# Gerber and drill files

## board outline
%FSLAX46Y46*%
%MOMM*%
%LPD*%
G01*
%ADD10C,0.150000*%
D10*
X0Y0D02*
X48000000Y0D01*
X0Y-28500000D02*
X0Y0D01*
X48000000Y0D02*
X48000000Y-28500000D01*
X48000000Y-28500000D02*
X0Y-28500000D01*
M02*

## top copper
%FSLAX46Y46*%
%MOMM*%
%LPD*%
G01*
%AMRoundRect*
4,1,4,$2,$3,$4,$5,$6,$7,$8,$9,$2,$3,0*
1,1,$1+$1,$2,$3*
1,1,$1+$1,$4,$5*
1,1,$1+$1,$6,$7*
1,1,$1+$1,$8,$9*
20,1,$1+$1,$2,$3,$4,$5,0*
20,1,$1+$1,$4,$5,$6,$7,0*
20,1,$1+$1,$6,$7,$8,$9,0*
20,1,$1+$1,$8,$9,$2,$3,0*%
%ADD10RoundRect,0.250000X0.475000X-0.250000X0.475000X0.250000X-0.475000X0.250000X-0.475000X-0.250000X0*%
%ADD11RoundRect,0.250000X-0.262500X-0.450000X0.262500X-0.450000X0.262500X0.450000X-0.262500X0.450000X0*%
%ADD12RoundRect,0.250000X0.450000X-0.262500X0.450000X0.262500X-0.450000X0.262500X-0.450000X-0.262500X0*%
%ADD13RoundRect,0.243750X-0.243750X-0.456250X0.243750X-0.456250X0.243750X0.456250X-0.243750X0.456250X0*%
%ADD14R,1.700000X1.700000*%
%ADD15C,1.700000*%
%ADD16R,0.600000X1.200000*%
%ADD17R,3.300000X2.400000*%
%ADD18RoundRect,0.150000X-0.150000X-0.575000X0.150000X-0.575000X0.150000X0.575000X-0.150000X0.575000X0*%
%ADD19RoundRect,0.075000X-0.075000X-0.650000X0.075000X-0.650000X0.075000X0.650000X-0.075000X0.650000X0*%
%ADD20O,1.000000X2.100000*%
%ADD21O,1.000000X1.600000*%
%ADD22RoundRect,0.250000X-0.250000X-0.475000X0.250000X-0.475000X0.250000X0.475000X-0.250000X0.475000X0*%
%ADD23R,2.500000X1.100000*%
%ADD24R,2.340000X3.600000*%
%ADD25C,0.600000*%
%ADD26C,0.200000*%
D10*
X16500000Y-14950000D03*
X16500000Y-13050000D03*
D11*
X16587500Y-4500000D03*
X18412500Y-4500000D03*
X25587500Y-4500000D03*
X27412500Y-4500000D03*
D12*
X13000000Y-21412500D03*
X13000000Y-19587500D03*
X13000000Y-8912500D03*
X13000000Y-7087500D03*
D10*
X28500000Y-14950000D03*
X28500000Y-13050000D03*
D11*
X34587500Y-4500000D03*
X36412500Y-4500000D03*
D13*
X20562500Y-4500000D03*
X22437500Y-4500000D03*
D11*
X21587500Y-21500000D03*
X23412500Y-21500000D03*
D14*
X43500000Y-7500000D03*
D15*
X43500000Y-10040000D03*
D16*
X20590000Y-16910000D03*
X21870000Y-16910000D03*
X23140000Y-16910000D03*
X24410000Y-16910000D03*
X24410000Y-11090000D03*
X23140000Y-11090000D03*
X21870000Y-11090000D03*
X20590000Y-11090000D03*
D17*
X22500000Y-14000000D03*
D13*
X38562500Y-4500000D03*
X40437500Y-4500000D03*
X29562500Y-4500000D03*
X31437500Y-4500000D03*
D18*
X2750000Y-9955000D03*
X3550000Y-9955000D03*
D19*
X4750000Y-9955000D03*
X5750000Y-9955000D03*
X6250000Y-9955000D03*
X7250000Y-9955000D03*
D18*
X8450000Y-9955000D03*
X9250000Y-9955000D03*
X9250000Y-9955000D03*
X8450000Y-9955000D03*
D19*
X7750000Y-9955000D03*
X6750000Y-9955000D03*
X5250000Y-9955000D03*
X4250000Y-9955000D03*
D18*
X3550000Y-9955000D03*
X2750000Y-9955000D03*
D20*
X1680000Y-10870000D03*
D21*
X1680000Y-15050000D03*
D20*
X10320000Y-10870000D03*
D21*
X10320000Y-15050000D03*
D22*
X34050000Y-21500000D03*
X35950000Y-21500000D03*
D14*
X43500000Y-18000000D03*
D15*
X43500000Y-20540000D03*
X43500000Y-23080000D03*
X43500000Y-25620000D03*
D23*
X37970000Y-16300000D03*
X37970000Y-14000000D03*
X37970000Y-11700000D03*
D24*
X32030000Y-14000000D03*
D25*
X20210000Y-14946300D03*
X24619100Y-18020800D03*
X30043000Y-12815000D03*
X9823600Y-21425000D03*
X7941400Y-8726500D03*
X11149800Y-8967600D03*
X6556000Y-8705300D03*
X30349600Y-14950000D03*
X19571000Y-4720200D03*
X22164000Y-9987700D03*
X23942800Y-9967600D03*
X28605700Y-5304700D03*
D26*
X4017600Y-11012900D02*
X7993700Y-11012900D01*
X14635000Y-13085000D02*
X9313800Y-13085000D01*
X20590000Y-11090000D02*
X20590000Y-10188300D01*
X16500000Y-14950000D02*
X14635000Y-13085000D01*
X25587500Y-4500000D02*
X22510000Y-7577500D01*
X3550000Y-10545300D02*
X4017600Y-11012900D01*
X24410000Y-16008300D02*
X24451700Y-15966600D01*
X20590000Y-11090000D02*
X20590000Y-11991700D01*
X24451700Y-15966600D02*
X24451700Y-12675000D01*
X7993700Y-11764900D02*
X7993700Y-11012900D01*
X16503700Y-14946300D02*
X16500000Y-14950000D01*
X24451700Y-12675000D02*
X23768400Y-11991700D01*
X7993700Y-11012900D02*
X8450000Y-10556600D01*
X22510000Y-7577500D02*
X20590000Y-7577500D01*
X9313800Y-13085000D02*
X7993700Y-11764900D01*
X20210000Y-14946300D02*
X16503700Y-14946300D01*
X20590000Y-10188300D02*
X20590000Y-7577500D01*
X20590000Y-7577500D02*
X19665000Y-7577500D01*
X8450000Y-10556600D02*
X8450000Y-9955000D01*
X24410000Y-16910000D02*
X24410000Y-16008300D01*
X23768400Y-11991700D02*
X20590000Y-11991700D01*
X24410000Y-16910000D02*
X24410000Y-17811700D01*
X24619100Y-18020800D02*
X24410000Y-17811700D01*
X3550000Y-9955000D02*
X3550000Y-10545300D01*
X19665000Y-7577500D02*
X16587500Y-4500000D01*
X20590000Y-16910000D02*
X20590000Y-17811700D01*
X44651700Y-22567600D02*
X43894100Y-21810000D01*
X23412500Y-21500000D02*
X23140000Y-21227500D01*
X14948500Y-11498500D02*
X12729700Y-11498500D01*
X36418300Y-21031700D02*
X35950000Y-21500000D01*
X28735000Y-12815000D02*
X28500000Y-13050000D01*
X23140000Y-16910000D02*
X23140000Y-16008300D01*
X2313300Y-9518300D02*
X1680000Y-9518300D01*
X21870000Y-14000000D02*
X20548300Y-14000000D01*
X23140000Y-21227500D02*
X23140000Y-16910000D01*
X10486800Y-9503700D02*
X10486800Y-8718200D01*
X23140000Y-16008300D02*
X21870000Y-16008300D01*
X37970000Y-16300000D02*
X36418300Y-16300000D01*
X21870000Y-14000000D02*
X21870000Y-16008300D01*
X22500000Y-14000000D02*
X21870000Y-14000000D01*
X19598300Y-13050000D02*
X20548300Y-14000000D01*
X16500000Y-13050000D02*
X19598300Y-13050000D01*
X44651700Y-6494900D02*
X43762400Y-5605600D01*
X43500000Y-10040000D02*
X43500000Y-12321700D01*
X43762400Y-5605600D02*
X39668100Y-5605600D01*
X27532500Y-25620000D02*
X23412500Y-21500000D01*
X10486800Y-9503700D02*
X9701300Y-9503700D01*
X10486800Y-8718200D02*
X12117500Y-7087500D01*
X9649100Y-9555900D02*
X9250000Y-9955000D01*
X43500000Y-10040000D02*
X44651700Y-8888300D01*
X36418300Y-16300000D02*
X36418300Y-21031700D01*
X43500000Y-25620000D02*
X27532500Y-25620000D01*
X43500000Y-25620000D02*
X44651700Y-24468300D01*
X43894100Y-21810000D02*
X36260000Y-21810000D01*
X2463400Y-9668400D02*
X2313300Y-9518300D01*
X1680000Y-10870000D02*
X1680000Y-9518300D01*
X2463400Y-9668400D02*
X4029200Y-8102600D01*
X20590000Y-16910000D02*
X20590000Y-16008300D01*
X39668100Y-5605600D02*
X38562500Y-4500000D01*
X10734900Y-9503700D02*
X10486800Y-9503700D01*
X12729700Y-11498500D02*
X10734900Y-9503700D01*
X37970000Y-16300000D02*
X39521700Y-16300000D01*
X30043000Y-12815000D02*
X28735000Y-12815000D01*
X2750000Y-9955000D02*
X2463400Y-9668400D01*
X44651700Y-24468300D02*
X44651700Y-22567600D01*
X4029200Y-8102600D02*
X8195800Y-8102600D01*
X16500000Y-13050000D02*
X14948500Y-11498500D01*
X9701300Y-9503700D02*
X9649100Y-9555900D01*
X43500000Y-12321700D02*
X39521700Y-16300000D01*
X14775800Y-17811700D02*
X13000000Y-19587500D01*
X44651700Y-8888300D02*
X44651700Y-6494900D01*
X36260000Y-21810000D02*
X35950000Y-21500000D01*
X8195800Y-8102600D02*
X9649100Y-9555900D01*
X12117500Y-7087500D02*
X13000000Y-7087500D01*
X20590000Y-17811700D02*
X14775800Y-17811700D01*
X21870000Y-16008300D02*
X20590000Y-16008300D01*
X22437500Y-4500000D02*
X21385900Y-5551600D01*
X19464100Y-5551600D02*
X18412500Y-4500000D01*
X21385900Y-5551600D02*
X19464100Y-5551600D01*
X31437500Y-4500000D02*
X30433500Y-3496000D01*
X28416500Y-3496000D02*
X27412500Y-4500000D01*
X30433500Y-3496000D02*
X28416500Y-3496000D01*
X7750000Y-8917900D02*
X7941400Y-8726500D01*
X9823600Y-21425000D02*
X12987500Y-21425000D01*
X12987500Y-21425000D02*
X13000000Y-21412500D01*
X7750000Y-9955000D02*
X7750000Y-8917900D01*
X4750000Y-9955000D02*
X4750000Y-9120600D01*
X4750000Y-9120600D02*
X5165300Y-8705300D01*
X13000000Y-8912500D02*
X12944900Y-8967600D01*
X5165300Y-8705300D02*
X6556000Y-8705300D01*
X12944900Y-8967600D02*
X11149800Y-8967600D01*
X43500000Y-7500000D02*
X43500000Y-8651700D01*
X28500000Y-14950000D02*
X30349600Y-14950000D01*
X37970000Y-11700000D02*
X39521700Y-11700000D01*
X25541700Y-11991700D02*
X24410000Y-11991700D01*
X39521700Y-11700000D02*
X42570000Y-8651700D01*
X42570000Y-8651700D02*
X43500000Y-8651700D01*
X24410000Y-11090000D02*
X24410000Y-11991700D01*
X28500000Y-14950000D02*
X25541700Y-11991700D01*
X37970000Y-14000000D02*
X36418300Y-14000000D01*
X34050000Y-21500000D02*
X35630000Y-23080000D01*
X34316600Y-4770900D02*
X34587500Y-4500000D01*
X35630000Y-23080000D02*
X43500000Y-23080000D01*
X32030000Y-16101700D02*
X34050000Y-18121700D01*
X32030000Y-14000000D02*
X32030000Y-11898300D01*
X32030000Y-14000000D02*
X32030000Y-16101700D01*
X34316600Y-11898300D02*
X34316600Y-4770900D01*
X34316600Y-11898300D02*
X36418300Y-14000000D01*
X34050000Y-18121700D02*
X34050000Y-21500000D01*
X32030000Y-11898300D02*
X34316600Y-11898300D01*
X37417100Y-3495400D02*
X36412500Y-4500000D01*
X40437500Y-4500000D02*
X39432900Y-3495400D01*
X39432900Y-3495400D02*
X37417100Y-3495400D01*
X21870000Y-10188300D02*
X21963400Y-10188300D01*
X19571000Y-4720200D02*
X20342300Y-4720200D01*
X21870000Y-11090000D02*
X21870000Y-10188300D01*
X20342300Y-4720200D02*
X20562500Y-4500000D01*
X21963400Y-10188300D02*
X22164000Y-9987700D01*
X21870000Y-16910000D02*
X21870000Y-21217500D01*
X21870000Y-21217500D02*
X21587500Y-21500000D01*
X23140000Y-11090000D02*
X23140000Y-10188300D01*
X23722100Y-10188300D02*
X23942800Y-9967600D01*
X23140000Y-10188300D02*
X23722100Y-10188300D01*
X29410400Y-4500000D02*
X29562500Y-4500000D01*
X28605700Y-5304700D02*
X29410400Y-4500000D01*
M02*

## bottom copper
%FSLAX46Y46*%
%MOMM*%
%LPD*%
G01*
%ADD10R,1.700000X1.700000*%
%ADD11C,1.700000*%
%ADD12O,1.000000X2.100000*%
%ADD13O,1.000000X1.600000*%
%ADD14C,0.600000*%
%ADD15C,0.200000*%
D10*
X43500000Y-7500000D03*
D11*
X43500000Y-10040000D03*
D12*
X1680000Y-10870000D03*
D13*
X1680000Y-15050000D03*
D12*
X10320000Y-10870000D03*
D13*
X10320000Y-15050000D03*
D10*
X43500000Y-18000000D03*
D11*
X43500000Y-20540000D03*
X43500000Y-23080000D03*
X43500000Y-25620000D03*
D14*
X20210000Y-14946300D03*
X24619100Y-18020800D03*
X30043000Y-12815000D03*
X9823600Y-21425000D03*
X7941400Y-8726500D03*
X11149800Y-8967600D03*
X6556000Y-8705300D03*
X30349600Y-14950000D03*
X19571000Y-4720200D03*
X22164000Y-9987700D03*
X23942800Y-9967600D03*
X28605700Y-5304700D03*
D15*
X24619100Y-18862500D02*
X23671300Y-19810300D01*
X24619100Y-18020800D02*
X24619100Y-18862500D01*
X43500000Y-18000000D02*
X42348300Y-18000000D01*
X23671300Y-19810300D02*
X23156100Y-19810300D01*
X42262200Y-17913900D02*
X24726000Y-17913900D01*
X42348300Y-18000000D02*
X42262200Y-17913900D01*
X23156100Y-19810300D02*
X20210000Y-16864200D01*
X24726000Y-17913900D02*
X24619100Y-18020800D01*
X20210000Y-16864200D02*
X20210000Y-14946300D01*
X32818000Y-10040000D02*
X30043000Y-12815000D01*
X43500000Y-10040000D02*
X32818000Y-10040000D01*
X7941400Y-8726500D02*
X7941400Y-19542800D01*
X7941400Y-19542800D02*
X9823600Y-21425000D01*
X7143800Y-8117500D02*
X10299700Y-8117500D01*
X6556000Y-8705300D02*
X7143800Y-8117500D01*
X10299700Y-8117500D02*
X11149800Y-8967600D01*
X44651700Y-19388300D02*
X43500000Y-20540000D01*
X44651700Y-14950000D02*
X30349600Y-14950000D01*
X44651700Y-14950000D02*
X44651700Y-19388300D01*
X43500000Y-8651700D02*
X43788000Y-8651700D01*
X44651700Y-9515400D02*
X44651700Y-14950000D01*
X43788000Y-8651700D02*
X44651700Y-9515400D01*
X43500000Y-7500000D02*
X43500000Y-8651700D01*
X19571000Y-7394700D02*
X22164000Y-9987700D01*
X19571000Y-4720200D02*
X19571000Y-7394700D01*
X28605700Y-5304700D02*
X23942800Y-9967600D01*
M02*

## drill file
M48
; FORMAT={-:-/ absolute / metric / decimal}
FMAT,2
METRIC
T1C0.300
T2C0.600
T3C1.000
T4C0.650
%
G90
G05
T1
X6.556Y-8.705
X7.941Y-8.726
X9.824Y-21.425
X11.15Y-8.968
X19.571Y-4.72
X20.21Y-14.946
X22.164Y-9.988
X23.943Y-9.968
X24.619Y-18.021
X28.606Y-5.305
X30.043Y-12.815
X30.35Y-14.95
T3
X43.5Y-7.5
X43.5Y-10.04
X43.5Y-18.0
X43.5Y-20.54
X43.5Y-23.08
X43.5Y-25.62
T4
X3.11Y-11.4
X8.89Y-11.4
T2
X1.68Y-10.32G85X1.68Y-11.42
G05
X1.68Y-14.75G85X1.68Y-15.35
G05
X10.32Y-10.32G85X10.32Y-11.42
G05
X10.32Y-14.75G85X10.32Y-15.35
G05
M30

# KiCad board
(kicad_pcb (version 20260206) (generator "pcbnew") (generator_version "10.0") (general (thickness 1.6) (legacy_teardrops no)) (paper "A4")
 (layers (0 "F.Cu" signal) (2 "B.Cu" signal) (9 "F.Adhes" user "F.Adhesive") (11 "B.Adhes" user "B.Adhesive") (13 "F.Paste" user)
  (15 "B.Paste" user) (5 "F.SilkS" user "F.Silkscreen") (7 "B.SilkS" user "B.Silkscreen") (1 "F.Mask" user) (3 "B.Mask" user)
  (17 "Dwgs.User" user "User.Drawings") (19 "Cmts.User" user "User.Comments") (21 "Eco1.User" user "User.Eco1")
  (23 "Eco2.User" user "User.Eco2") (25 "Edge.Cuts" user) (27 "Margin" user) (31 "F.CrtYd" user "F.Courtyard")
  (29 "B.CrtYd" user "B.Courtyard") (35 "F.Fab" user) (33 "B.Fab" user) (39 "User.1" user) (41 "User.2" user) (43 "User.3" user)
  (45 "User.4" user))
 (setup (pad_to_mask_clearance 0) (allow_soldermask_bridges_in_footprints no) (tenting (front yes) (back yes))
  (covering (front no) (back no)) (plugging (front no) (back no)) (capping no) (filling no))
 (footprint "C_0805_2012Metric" (layer "F.Cu") (at 16.5 14 90)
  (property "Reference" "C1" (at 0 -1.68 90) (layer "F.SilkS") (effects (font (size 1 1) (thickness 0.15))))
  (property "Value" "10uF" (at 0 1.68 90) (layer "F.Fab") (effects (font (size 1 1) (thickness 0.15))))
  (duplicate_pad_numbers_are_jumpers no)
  (pad "1" smd roundrect (at -0.95 0 90) (size 1 1.45) (layers "F.Cu" "F.Mask" "F.Paste") (roundrect_rratio 0.25) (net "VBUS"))
  (pad "2" smd roundrect (at 0.95 0 90) (size 1 1.45) (layers "F.Cu" "F.Mask" "F.Paste") (roundrect_rratio 0.25) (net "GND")))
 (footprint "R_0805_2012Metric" (layer "F.Cu") (at 17.5 4.5)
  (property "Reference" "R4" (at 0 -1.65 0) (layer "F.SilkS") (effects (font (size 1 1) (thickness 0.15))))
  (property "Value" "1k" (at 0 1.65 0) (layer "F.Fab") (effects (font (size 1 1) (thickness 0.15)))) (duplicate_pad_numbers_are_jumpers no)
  (pad "1" smd roundrect (at -0.9125 0) (size 1.025 1.4) (layers "F.Cu" "F.Mask" "F.Paste") (roundrect_rratio 0.243902) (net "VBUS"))
  (pad "2" smd roundrect (at 0.9125 0) (size 1.025 1.4) (layers "F.Cu" "F.Mask" "F.Paste") (roundrect_rratio 0.243902) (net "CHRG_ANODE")))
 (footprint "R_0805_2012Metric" (layer "F.Cu") (at 26.5 4.5)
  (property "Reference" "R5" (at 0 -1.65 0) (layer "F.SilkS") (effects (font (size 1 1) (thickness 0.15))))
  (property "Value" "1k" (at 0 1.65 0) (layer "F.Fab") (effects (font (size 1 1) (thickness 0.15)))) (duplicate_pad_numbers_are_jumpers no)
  (pad "1" smd roundrect (at -0.9125 0) (size 1.025 1.4) (layers "F.Cu" "F.Mask" "F.Paste") (roundrect_rratio 0.243902) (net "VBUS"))
  (pad "2" smd roundrect (at 0.9125 0) (size 1.025 1.4) (layers "F.Cu" "F.Mask" "F.Paste") (roundrect_rratio 0.243902) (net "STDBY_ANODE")))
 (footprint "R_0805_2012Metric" (layer "F.Cu") (at 13 20.5 90)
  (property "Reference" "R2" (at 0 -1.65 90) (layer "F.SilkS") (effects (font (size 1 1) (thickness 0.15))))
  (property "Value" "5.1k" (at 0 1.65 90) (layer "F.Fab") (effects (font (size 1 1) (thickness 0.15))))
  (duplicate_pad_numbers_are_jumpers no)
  (pad "1" smd roundrect (at -0.9125 0 90) (size 1.025 1.4) (layers "F.Cu" "F.Mask" "F.Paste") (roundrect_rratio 0.243902) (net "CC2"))
  (pad "2" smd roundrect (at 0.9125 0 90) (size 1.025 1.4) (layers "F.Cu" "F.Mask" "F.Paste") (roundrect_rratio 0.243902) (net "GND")))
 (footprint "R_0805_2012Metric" (layer "F.Cu") (at 13 8 90)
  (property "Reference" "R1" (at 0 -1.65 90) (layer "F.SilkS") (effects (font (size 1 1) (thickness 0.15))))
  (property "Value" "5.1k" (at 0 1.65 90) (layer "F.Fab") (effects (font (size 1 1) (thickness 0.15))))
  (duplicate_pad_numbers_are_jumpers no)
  (pad "1" smd roundrect (at -0.9125 0 90) (size 1.025 1.4) (layers "F.Cu" "F.Mask" "F.Paste") (roundrect_rratio 0.243902) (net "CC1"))
  (pad "2" smd roundrect (at 0.9125 0 90) (size 1.025 1.4) (layers "F.Cu" "F.Mask" "F.Paste") (roundrect_rratio 0.243902) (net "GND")))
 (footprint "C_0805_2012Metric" (layer "F.Cu") (at 28.5 14 90)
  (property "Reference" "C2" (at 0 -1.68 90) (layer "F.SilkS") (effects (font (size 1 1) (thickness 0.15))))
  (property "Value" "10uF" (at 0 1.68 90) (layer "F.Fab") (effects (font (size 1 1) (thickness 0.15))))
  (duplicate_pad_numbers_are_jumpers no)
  (pad "1" smd roundrect (at -0.95 0 90) (size 1 1.45) (layers "F.Cu" "F.Mask" "F.Paste") (roundrect_rratio 0.25) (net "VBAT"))
  (pad "2" smd roundrect (at 0.95 0 90) (size 1 1.45) (layers "F.Cu" "F.Mask" "F.Paste") (roundrect_rratio 0.25) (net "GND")))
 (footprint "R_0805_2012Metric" (layer "F.Cu") (at 35.5 4.5)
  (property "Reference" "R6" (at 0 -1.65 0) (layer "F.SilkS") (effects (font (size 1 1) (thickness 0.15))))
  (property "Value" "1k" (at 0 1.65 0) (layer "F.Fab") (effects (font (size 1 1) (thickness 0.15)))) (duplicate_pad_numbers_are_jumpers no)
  (pad "1" smd roundrect (at -0.9125 0) (size 1.025 1.4) (layers "F.Cu" "F.Mask" "F.Paste") (roundrect_rratio 0.243902) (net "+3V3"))
  (pad "2" smd roundrect (at 0.9125 0) (size 1.025 1.4) (layers "F.Cu" "F.Mask" "F.Paste") (roundrect_rratio 0.243902) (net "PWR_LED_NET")))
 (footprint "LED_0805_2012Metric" (layer "F.Cu") (at 21.5 4.5)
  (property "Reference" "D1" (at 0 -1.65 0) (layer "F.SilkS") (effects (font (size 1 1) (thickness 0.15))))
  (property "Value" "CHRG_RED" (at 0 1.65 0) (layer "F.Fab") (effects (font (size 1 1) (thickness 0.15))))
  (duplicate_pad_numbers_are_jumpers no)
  (pad "1" smd roundrect (at -0.9375 0) (size 0.975 1.4) (layers "F.Cu" "F.Mask" "F.Paste") (roundrect_rratio 0.25) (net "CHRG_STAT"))
  (pad "2" smd roundrect (at 0.9375 0) (size 0.975 1.4) (layers "F.Cu" "F.Mask" "F.Paste") (roundrect_rratio 0.25) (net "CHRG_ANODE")))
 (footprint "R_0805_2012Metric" (layer "F.Cu") (at 22.5 21.5)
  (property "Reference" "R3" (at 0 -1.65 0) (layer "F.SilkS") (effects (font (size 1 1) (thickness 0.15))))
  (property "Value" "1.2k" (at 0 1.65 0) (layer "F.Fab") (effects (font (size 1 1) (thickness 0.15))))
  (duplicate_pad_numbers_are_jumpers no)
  (pad "1" smd roundrect (at -0.9125 0) (size 1.025 1.4) (layers "F.Cu" "F.Mask" "F.Paste") (roundrect_rratio 0.243902) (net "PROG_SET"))
  (pad "2" smd roundrect (at 0.9125 0) (size 1.025 1.4) (layers "F.Cu" "F.Mask" "F.Paste") (roundrect_rratio 0.243902) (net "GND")))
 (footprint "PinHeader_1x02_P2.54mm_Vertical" (layer "F.Cu") (at 43.5 7.5)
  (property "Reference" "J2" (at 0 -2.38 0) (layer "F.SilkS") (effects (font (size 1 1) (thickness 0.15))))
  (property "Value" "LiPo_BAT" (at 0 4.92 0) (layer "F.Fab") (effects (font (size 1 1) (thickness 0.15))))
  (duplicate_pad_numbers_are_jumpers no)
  (pad "1" thru_hole rect (at 0 0) (size 1.7 1.7) (drill 1) (layers "*.Cu" "*.Mask") (remove_unused_layers no) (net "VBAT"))
  (pad "2" thru_hole circle (at 0 2.54) (size 1.7 1.7) (drill 1) (layers "*.Cu" "*.Mask") (remove_unused_layers no) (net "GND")))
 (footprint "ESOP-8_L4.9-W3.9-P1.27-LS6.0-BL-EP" (layer "F.Cu") (at 22.5 14)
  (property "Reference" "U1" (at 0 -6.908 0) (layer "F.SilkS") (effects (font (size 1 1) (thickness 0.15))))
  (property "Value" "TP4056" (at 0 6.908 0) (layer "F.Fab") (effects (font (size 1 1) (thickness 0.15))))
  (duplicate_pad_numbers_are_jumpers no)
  (pad "1" smd rect (at -1.91 2.91) (size 0.6 1.2) (layers "F.Cu" "F.Mask" "F.Paste") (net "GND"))
  (pad "2" smd rect (at -0.63 2.91) (size 0.6 1.2) (layers "F.Cu" "F.Mask" "F.Paste") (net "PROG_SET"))
  (pad "3" smd rect (at 0.64 2.91) (size 0.6 1.2) (layers "F.Cu" "F.Mask" "F.Paste") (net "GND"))
  (pad "4" smd rect (at 1.91 2.91) (size 0.6 1.2) (layers "F.Cu" "F.Mask" "F.Paste") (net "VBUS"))
  (pad "5" smd rect (at 1.91 -2.91) (size 0.6 1.2) (layers "F.Cu" "F.Mask" "F.Paste") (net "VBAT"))
  (pad "6" smd rect (at 0.64 -2.91) (size 0.6 1.2) (layers "F.Cu" "F.Mask" "F.Paste") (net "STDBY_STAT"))
  (pad "7" smd rect (at -0.63 -2.91) (size 0.6 1.2) (layers "F.Cu" "F.Mask" "F.Paste") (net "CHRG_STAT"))
  (pad "8" smd rect (at -1.91 -2.91) (size 0.6 1.2) (layers "F.Cu" "F.Mask" "F.Paste") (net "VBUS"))
  (pad "9" smd rect (at 0 0 180) (size 3.3 2.4) (layers "F.Cu" "F.Mask" "F.Paste") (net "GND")))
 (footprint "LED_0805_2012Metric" (layer "F.Cu") (at 39.5 4.5)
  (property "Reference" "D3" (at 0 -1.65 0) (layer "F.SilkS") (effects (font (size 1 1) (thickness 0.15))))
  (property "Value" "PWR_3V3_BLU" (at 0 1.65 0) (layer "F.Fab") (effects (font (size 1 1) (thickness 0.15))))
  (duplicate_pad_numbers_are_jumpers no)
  (pad "1" smd roundrect (at -0.9375 0) (size 0.975 1.4) (layers "F.Cu" "F.Mask" "F.Paste") (roundrect_rratio 0.25) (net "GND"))
  (pad "2" smd roundrect (at 0.9375 0) (size 0.975 1.4) (layers "F.Cu" "F.Mask" "F.Paste") (roundrect_rratio 0.25) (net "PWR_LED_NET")))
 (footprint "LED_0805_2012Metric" (layer "F.Cu") (at 30.5 4.5)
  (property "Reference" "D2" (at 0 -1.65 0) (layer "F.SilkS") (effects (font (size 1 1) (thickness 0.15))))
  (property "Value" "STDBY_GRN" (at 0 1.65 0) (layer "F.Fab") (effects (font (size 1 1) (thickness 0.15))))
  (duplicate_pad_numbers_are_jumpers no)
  (pad "1" smd roundrect (at -0.9375 0) (size 0.975 1.4) (layers "F.Cu" "F.Mask" "F.Paste") (roundrect_rratio 0.25) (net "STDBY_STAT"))
  (pad "2" smd roundrect (at 0.9375 0) (size 0.975 1.4) (layers "F.Cu" "F.Mask" "F.Paste") (roundrect_rratio 0.25) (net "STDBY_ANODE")))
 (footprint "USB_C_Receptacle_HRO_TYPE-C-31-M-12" (layer "F.Cu") (at 6 14)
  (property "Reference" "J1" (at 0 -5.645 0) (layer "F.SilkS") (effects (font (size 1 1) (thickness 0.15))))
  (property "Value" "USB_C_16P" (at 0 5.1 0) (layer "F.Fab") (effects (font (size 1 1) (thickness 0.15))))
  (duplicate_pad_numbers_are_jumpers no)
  (pad "" np_thru_hole circle (at -2.89 -2.6) (size 0.65 0.65) (drill 0.65) (layers "*.Cu" "*.Mask"))
  (pad "" np_thru_hole circle (at 2.89 -2.6) (size 0.65 0.65) (drill 0.65) (layers "*.Cu" "*.Mask"))
  (pad "A1" smd roundrect (at -3.25 -4.045) (size 0.6 1.45) (layers "F.Cu" "F.Mask" "F.Paste") (roundrect_rratio 0.25) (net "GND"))
  (pad "A4" smd roundrect (at -2.45 -4.045) (size 0.6 1.45) (layers "F.Cu" "F.Mask" "F.Paste") (roundrect_rratio 0.25) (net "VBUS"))
  (pad "A5" smd roundrect (at -1.25 -4.045) (size 0.3 1.45) (layers "F.Cu" "F.Mask" "F.Paste") (roundrect_rratio 0.25) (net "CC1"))
  (pad "A6" smd roundrect (at -0.25 -4.045) (size 0.3 1.45) (layers "F.Cu" "F.Mask" "F.Paste") (roundrect_rratio 0.25))
  (pad "A7" smd roundrect (at 0.25 -4.045) (size 0.3 1.45) (layers "F.Cu" "F.Mask" "F.Paste") (roundrect_rratio 0.25))
  (pad "A8" smd roundrect (at 1.25 -4.045) (size 0.3 1.45) (layers "F.Cu" "F.Mask" "F.Paste") (roundrect_rratio 0.25))
  (pad "A9" smd roundrect (at 2.45 -4.045) (size 0.6 1.45) (layers "F.Cu" "F.Mask" "F.Paste") (roundrect_rratio 0.25) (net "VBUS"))
  (pad "A12" smd roundrect (at 3.25 -4.045) (size 0.6 1.45) (layers "F.Cu" "F.Mask" "F.Paste") (roundrect_rratio 0.25) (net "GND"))
  (pad "B1" smd roundrect (at 3.25 -4.045) (size 0.6 1.45) (layers "F.Cu" "F.Mask" "F.Paste") (roundrect_rratio 0.25) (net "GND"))
  (pad "B4" smd roundrect (at 2.45 -4.045) (size 0.6 1.45) (layers "F.Cu" "F.Mask" "F.Paste") (roundrect_rratio 0.25) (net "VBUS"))
  (pad "B5" smd roundrect (at 1.75 -4.045) (size 0.3 1.45) (layers "F.Cu" "F.Mask" "F.Paste") (roundrect_rratio 0.25) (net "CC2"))
  (pad "B6" smd roundrect (at 0.75 -4.045) (size 0.3 1.45) (layers "F.Cu" "F.Mask" "F.Paste") (roundrect_rratio 0.25))
  (pad "B7" smd roundrect (at -0.75 -4.045) (size 0.3 1.45) (layers "F.Cu" "F.Mask" "F.Paste") (roundrect_rratio 0.25))
  (pad "B8" smd roundrect (at -1.75 -4.045) (size 0.3 1.45) (layers "F.Cu" "F.Mask" "F.Paste") (roundrect_rratio 0.25))
  (pad "B9" smd roundrect (at -2.45 -4.045) (size 0.6 1.45) (layers "F.Cu" "F.Mask" "F.Paste") (roundrect_rratio 0.25) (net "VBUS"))
  (pad "B12" smd roundrect (at -3.25 -4.045) (size 0.6 1.45) (layers "F.Cu" "F.Mask" "F.Paste") (roundrect_rratio 0.25) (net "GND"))
  (pad "SH" thru_hole oval (at -4.32 -3.13) (size 1 2.1) (drill oval 0.6 1.7) (layers "*.Cu" "*.Mask") (remove_unused_layers no) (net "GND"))
  (pad "SH" thru_hole oval (at -4.32 1.05) (size 1 1.6) (drill oval 0.6 1.2) (layers "*.Cu" "*.Mask") (remove_unused_layers no))
  (pad "SH" thru_hole oval (at 4.32 -3.13) (size 1 2.1) (drill oval 0.6 1.7) (layers "*.Cu" "*.Mask") (remove_unused_layers no))
  (pad "SH" thru_hole oval (at 4.32 1.05) (size 1 1.6) (drill oval 0.6 1.2) (layers "*.Cu" "*.Mask") (remove_unused_layers no)))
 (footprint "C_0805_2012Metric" (layer "F.Cu") (at 35 21.5)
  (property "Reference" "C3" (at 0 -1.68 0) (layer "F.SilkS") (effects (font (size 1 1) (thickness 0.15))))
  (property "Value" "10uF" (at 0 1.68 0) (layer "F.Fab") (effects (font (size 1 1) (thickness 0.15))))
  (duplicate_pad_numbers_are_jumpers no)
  (pad "1" smd roundrect (at -0.95 0) (size 1 1.45) (layers "F.Cu" "F.Mask" "F.Paste") (roundrect_rratio 0.25) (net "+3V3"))
  (pad "2" smd roundrect (at 0.95 0) (size 1 1.45) (layers "F.Cu" "F.Mask" "F.Paste") (roundrect_rratio 0.25) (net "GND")))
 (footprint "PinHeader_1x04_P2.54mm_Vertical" (layer "F.Cu") (at 43.5 18)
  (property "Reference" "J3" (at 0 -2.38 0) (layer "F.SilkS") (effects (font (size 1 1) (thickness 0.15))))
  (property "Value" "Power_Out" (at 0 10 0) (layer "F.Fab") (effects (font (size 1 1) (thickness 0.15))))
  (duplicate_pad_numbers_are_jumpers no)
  (pad "1" thru_hole rect (at 0 0) (size 1.7 1.7) (drill 1) (layers "*.Cu" "*.Mask") (remove_unused_layers no) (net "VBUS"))
  (pad "2" thru_hole circle (at 0 2.54) (size 1.7 1.7) (drill 1) (layers "*.Cu" "*.Mask") (remove_unused_layers no) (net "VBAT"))
  (pad "3" thru_hole circle (at 0 5.08) (size 1.7 1.7) (drill 1) (layers "*.Cu" "*.Mask") (remove_unused_layers no) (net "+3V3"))
  (pad "4" thru_hole circle (at 0 7.62) (size 1.7 1.7) (drill 1) (layers "*.Cu" "*.Mask") (remove_unused_layers no) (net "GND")))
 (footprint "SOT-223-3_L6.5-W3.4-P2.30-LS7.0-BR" (layer "F.Cu") (at 35 14)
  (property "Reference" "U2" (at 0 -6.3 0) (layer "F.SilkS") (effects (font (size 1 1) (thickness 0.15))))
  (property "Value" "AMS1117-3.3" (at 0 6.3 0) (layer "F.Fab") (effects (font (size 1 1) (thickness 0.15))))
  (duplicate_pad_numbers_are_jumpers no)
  (pad "1" smd rect (at 2.97 2.3) (size 2.5 1.1) (layers "F.Cu" "F.Mask" "F.Paste") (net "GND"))
  (pad "2" smd rect (at 2.97 0) (size 2.5 1.1) (layers "F.Cu" "F.Mask" "F.Paste") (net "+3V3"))
  (pad "3" smd rect (at 2.97 -2.3) (size 2.5 1.1) (layers "F.Cu" "F.Mask" "F.Paste") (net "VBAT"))
  (pad "4" smd rect (at -2.97 0) (size 2.34 3.6) (layers "F.Cu" "F.Mask" "F.Paste") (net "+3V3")))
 (gr_line (start 0 0) (end 48 0) (stroke (width 0.15) (type default)) (layer "Edge.Cuts"))
 (gr_line (start 0 28.5) (end 0 0) (stroke (width 0.15) (type default)) (layer "Edge.Cuts"))
 (gr_line (start 48 0) (end 48 28.5) (stroke (width 0.15) (type default)) (layer "Edge.Cuts"))
 (gr_line (start 48 28.5) (end 0 28.5) (stroke (width 0.15) (type default)) (layer "Edge.Cuts"))
 (segment (start 4.0176 11.0129) (end 7.9937 11.0129) (width 0.2) (layer "F.Cu") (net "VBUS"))
 (segment (start 14.635 13.085) (end 9.3138 13.085) (width 0.2) (layer "F.Cu") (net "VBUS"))
 (segment (start 20.59 11.09) (end 20.59 10.1883) (width 0.2) (layer "F.Cu") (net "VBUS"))
 (segment (start 16.5 14.95) (end 14.635 13.085) (width 0.2) (layer "F.Cu") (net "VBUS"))
 (segment (start 25.5875 4.5) (end 22.51 7.5775) (width 0.2) (layer "F.Cu") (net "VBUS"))
 (segment (start 3.55 10.5453) (end 4.0176 11.0129) (width 0.2) (layer "F.Cu") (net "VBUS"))
 (segment (start 24.41 16.0083) (end 24.4517 15.9666) (width 0.2) (layer "F.Cu") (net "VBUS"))
 (segment (start 20.59 11.09) (end 20.59 11.9917) (width 0.2) (layer "F.Cu") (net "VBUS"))
 (segment (start 24.4517 15.9666) (end 24.4517 12.675) (width 0.2) (layer "F.Cu") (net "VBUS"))
 (segment (start 7.9937 11.7649) (end 7.9937 11.0129) (width 0.2) (layer "F.Cu") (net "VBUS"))
 (segment (start 16.5037 14.9463) (end 16.5 14.95) (width 0.2) (layer "F.Cu") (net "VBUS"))
 (segment (start 24.4517 12.675) (end 23.7684 11.9917) (width 0.2) (layer "F.Cu") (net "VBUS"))
 (segment (start 7.9937 11.0129) (end 8.45 10.5566) (width 0.2) (layer "F.Cu") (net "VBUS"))
 (segment (start 22.51 7.5775) (end 20.59 7.5775) (width 0.2) (layer "F.Cu") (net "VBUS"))
 (segment (start 9.3138 13.085) (end 7.9937 11.7649) (width 0.2) (layer "F.Cu") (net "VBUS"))
 (segment (start 20.21 14.9463) (end 16.5037 14.9463) (width 0.2) (layer "F.Cu") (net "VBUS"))
 (segment (start 20.59 10.1883) (end 20.59 7.5775) (width 0.2) (layer "F.Cu") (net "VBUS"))
 (segment (start 20.59 7.5775) (end 19.665 7.5775) (width 0.2) (layer "F.Cu") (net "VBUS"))
 (segment (start 8.45 10.5566) (end 8.45 9.955) (width 0.2) (layer "F.Cu") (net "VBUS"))
 (segment (start 24.41 16.91) (end 24.41 16.0083) (width 0.2) (layer "F.Cu") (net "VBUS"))
 (segment (start 23.7684 11.9917) (end 20.59 11.9917) (width 0.2) (layer "F.Cu") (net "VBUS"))
 (segment (start 24.41 16.91) (end 24.41 17.8117) (width 0.2) (layer "F.Cu") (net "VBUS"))
 (segment (start 24.6191 18.0208) (end 24.41 17.8117) (width 0.2) (layer "F.Cu") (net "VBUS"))
 (segment (start 3.55 9.955) (end 3.55 10.5453) (width 0.2) (layer "F.Cu") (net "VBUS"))
 (segment (start 19.665 7.5775) (end 16.5875 4.5) (width 0.2) (layer "F.Cu") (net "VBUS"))
 (via (at 20.21 14.9463) (size 0.6) (drill 0.3) (layers "F.Cu" "B.Cu") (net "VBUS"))
 (via (at 24.6191 18.0208) (size 0.6) (drill 0.3) (layers "F.Cu" "B.Cu") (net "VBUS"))
 (segment (start 24.6191 18.8625) (end 23.6713 19.8103) (width 0.2) (layer "B.Cu") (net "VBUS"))
 (segment (start 24.6191 18.0208) (end 24.6191 18.8625) (width 0.2) (layer "B.Cu") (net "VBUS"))
 (segment (start 43.5 18) (end 42.3483 18) (width 0.2) (layer "B.Cu") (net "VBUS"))
 (segment (start 23.6713 19.8103) (end 23.1561 19.8103) (width 0.2) (layer "B.Cu") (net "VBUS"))
 (segment (start 42.2622 17.9139) (end 24.726 17.9139) (width 0.2) (layer "B.Cu") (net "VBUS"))
 (segment (start 42.3483 18) (end 42.2622 17.9139) (width 0.2) (layer "B.Cu") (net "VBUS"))
 (segment (start 23.1561 19.8103) (end 20.21 16.8642) (width 0.2) (layer "B.Cu") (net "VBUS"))
 (segment (start 24.726 17.9139) (end 24.6191 18.0208) (width 0.2) (layer "B.Cu") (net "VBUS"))
 (segment (start 20.21 16.8642) (end 20.21 14.9463) (width 0.2) (layer "B.Cu") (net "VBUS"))
 (segment (start 20.59 16.91) (end 20.59 17.8117) (width 0.2) (layer "F.Cu") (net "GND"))
 (segment (start 44.6517 22.5676) (end 43.8941 21.81) (width 0.2) (layer "F.Cu") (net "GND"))
 (segment (start 23.4125 21.5) (end 23.14 21.2275) (width 0.2) (layer "F.Cu") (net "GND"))
 (segment (start 14.9485 11.4985) (end 12.7297 11.4985) (width 0.2) (layer "F.Cu") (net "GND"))
 (segment (start 36.4183 21.0317) (end 35.95 21.5) (width 0.2) (layer "F.Cu") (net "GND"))
 (segment (start 28.735 12.815) (end 28.5 13.05) (width 0.2) (layer "F.Cu") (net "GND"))
 (segment (start 23.14 16.91) (end 23.14 16.0083) (width 0.2) (layer "F.Cu") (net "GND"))
 (segment (start 2.3133 9.5183) (end 1.68 9.5183) (width 0.2) (layer "F.Cu") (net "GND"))
 (segment (start 21.87 14) (end 20.5483 14) (width 0.2) (layer "F.Cu") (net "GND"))
 (segment (start 23.14 21.2275) (end 23.14 16.91) (width 0.2) (layer "F.Cu") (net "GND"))
 (segment (start 10.4868 9.5037) (end 10.4868 8.7182) (width 0.2) (layer "F.Cu") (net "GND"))
 (segment (start 23.14 16.0083) (end 21.87 16.0083) (width 0.2) (layer "F.Cu") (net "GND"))
 (segment (start 37.97 16.3) (end 36.4183 16.3) (width 0.2) (layer "F.Cu") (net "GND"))
 (segment (start 21.87 14) (end 21.87 16.0083) (width 0.2) (layer "F.Cu") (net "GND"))
 (segment (start 22.5 14) (end 21.87 14) (width 0.2) (layer "F.Cu") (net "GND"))
 (segment (start 19.5983 13.05) (end 20.5483 14) (width 0.2) (layer "F.Cu") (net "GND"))
 (segment (start 16.5 13.05) (end 19.5983 13.05) (width 0.2) (layer "F.Cu") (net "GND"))
 (segment (start 44.6517 6.4949) (end 43.7624 5.6056) (width 0.2) (layer "F.Cu") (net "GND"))
 (segment (start 43.5 10.04) (end 43.5 12.3217) (width 0.2) (layer "F.Cu") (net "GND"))
 (segment (start 43.7624 5.6056) (end 39.6681 5.6056) (width 0.2) (layer "F.Cu") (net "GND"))
 (segment (start 27.5325 25.62) (end 23.4125 21.5) (width 0.2) (layer "F.Cu") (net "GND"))
 (segment (start 10.4868 9.5037) (end 9.7013 9.5037) (width 0.2) (layer "F.Cu") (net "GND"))
 (segment (start 10.4868 8.7182) (end 12.1175 7.0875) (width 0.2) (layer "F.Cu") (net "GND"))
 (segment (start 9.6491 9.5559) (end 9.25 9.955) (width 0.2) (layer "F.Cu") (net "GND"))
 (segment (start 43.5 10.04) (end 44.6517 8.8883) (width 0.2) (layer "F.Cu") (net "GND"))
 (segment (start 36.4183 16.3) (end 36.4183 21.0317) (width 0.2) (layer "F.Cu") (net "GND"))
 (segment (start 43.5 25.62) (end 27.5325 25.62) (width 0.2) (layer "F.Cu") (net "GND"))
 (segment (start 43.5 25.62) (end 44.6517 24.4683) (width 0.2) (layer "F.Cu") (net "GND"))
 (segment (start 43.8941 21.81) (end 36.26 21.81) (width 0.2) (layer "F.Cu") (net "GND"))
 (segment (start 2.4634 9.6684) (end 2.3133 9.5183) (width 0.2) (layer "F.Cu") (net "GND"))
 (segment (start 1.68 10.87) (end 1.68 9.5183) (width 0.2) (layer "F.Cu") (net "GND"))
 (segment (start 2.4634 9.6684) (end 4.0292 8.1026) (width 0.2) (layer "F.Cu") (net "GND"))
 (segment (start 20.59 16.91) (end 20.59 16.0083) (width 0.2) (layer "F.Cu") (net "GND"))
 (segment (start 39.6681 5.6056) (end 38.5625 4.5) (width 0.2) (layer "F.Cu") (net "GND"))
 (segment (start 10.7349 9.5037) (end 10.4868 9.5037) (width 0.2) (layer "F.Cu") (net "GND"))
 (segment (start 12.7297 11.4985) (end 10.7349 9.5037) (width 0.2) (layer "F.Cu") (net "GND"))
 (segment (start 37.97 16.3) (end 39.5217 16.3) (width 0.2) (layer "F.Cu") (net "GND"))
 (segment (start 30.043 12.815) (end 28.735 12.815) (width 0.2) (layer "F.Cu") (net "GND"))
 (segment (start 2.75 9.955) (end 2.4634 9.6684) (width 0.2) (layer "F.Cu") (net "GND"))
 (segment (start 44.6517 24.4683) (end 44.6517 22.5676) (width 0.2) (layer "F.Cu") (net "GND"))
 (segment (start 4.0292 8.1026) (end 8.1958 8.1026) (width 0.2) (layer "F.Cu") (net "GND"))
 (segment (start 16.5 13.05) (end 14.9485 11.4985) (width 0.2) (layer "F.Cu") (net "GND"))
 (segment (start 9.7013 9.5037) (end 9.6491 9.5559) (width 0.2) (layer "F.Cu") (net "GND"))
 (segment (start 43.5 12.3217) (end 39.5217 16.3) (width 0.2) (layer "F.Cu") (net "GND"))
 (segment (start 14.7758 17.8117) (end 13 19.5875) (width 0.2) (layer "F.Cu") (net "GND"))
 (segment (start 44.6517 8.8883) (end 44.6517 6.4949) (width 0.2) (layer "F.Cu") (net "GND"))
 (segment (start 36.26 21.81) (end 35.95 21.5) (width 0.2) (layer "F.Cu") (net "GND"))
 (segment (start 8.1958 8.1026) (end 9.6491 9.5559) (width 0.2) (layer "F.Cu") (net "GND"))
 (segment (start 12.1175 7.0875) (end 13 7.0875) (width 0.2) (layer "F.Cu") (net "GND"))
 (segment (start 20.59 17.8117) (end 14.7758 17.8117) (width 0.2) (layer "F.Cu") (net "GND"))
 (segment (start 21.87 16.0083) (end 20.59 16.0083) (width 0.2) (layer "F.Cu") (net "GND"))
 (via (at 30.043 12.815) (size 0.6) (drill 0.3) (layers "F.Cu" "B.Cu") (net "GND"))
 (segment (start 32.818 10.04) (end 30.043 12.815) (width 0.2) (layer "B.Cu") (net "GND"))
 (segment (start 43.5 10.04) (end 32.818 10.04) (width 0.2) (layer "B.Cu") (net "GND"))
 (segment (start 22.4375 4.5) (end 21.3859 5.5516) (width 0.2) (layer "F.Cu") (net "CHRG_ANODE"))
 (segment (start 19.4641 5.5516) (end 18.4125 4.5) (width 0.2) (layer "F.Cu") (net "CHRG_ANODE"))
 (segment (start 21.3859 5.5516) (end 19.4641 5.5516) (width 0.2) (layer "F.Cu") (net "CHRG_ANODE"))
 (segment (start 31.4375 4.5) (end 30.4335 3.496) (width 0.2) (layer "F.Cu") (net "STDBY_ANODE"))
 (segment (start 28.4165 3.496) (end 27.4125 4.5) (width 0.2) (layer "F.Cu") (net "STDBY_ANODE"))
 (segment (start 30.4335 3.496) (end 28.4165 3.496) (width 0.2) (layer "F.Cu") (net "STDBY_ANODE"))
 (segment (start 7.75 8.9179) (end 7.9414 8.7265) (width 0.2) (layer "F.Cu") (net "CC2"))
 (segment (start 9.8236 21.425) (end 12.9875 21.425) (width 0.2) (layer "F.Cu") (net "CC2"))
 (segment (start 12.9875 21.425) (end 13 21.4125) (width 0.2) (layer "F.Cu") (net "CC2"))
 (segment (start 7.75 9.955) (end 7.75 8.9179) (width 0.2) (layer "F.Cu") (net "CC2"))
 (via (at 9.8236 21.425) (size 0.6) (drill 0.3) (layers "F.Cu" "B.Cu") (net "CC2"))
 (via (at 7.9414 8.7265) (size 0.6) (drill 0.3) (layers "F.Cu" "B.Cu") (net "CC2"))
 (segment (start 7.9414 8.7265) (end 7.9414 19.5428) (width 0.2) (layer "B.Cu") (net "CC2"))
 (segment (start 7.9414 19.5428) (end 9.8236 21.425) (width 0.2) (layer "B.Cu") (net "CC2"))
 (segment (start 4.75 9.955) (end 4.75 9.1206) (width 0.2) (layer "F.Cu") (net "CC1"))
 (segment (start 4.75 9.1206) (end 5.1653 8.7053) (width 0.2) (layer "F.Cu") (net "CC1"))
 (segment (start 13 8.9125) (end 12.9449 8.9676) (width 0.2) (layer "F.Cu") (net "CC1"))
 (segment (start 5.1653 8.7053) (end 6.556 8.7053) (width 0.2) (layer "F.Cu") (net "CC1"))
 (segment (start 12.9449 8.9676) (end 11.1498 8.9676) (width 0.2) (layer "F.Cu") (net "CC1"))
 (via (at 11.1498 8.9676) (size 0.6) (drill 0.3) (layers "F.Cu" "B.Cu") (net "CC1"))
 (via (at 6.556 8.7053) (size 0.6) (drill 0.3) (layers "F.Cu" "B.Cu") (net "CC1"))
 (segment (start 7.1438 8.1175) (end 10.2997 8.1175) (width 0.2) (layer "B.Cu") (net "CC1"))
 (segment (start 6.556 8.7053) (end 7.1438 8.1175) (width 0.2) (layer "B.Cu") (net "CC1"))
 (segment (start 10.2997 8.1175) (end 11.1498 8.9676) (width 0.2) (layer "B.Cu") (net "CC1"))
 (segment (start 43.5 7.5) (end 43.5 8.6517) (width 0.2) (layer "F.Cu") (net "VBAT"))
 (segment (start 28.5 14.95) (end 30.3496 14.95) (width 0.2) (layer "F.Cu") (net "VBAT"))
 (segment (start 37.97 11.7) (end 39.5217 11.7) (width 0.2) (layer "F.Cu") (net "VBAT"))
 (segment (start 25.5417 11.9917) (end 24.41 11.9917) (width 0.2) (layer "F.Cu") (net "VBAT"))
 (segment (start 39.5217 11.7) (end 42.57 8.6517) (width 0.2) (layer "F.Cu") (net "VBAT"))
 (segment (start 42.57 8.6517) (end 43.5 8.6517) (width 0.2) (layer "F.Cu") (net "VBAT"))
 (segment (start 24.41 11.09) (end 24.41 11.9917) (width 0.2) (layer "F.Cu") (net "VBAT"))
 (segment (start 28.5 14.95) (end 25.5417 11.9917) (width 0.2) (layer "F.Cu") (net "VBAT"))
 (via (at 30.3496 14.95) (size 0.6) (drill 0.3) (layers "F.Cu" "B.Cu") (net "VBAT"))
 (segment (start 44.6517 19.3883) (end 43.5 20.54) (width 0.2) (layer "B.Cu") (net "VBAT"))
 (segment (start 44.6517 14.95) (end 30.3496 14.95) (width 0.2) (layer "B.Cu") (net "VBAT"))
 (segment (start 44.6517 14.95) (end 44.6517 19.3883) (width 0.2) (layer "B.Cu") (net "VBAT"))
 (segment (start 43.5 8.6517) (end 43.788 8.6517) (width 0.2) (layer "B.Cu") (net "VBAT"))
 (segment (start 44.6517 9.5154) (end 44.6517 14.95) (width 0.2) (layer "B.Cu") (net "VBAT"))
 (segment (start 43.788 8.6517) (end 44.6517 9.5154) (width 0.2) (layer "B.Cu") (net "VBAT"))
 (segment (start 43.5 7.5) (end 43.5 8.6517) (width 0.2) (layer "B.Cu") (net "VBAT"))
 (segment (start 37.97 14) (end 36.4183 14) (width 0.2) (layer "F.Cu") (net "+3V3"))
 (segment (start 34.05 21.5) (end 35.63 23.08) (width 0.2) (layer "F.Cu") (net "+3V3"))
 (segment (start 34.3166 4.7709) (end 34.5875 4.5) (width 0.2) (layer "F.Cu") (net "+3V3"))
 (segment (start 35.63 23.08) (end 43.5 23.08) (width 0.2) (layer "F.Cu") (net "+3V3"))
 (segment (start 32.03 16.1017) (end 34.05 18.1217) (width 0.2) (layer "F.Cu") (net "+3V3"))
 (segment (start 32.03 14) (end 32.03 11.8983) (width 0.2) (layer "F.Cu") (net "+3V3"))
 (segment (start 32.03 14) (end 32.03 16.1017) (width 0.2) (layer "F.Cu") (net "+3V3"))
 (segment (start 34.3166 11.8983) (end 34.3166 4.7709) (width 0.2) (layer "F.Cu") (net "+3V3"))
 (segment (start 34.3166 11.8983) (end 36.4183 14) (width 0.2) (layer "F.Cu") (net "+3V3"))
 (segment (start 34.05 18.1217) (end 34.05 21.5) (width 0.2) (layer "F.Cu") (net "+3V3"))
 (segment (start 32.03 11.8983) (end 34.3166 11.8983) (width 0.2) (layer "F.Cu") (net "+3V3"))
 (segment (start 37.4171 3.4954) (end 36.4125 4.5) (width 0.2) (layer "F.Cu") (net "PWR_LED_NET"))
 (segment (start 40.4375 4.5) (end 39.4329 3.4954) (width 0.2) (layer "F.Cu") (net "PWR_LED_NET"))
 (segment (start 39.4329 3.4954) (end 37.4171 3.4954) (width 0.2) (layer "F.Cu") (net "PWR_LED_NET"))
 (segment (start 21.87 10.1883) (end 21.9634 10.1883) (width 0.2) (layer "F.Cu") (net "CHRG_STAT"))
 (segment (start 19.571 4.7202) (end 20.3423 4.7202) (width 0.2) (layer "F.Cu") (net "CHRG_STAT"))
 (segment (start 21.87 11.09) (end 21.87 10.1883) (width 0.2) (layer "F.Cu") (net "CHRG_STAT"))
 (segment (start 20.3423 4.7202) (end 20.5625 4.5) (width 0.2) (layer "F.Cu") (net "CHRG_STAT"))
 (segment (start 21.9634 10.1883) (end 22.164 9.9877) (width 0.2) (layer "F.Cu") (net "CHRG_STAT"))
 (via (at 19.571 4.7202) (size 0.6) (drill 0.3) (layers "F.Cu" "B.Cu") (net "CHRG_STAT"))
 (via (at 22.164 9.9877) (size 0.6) (drill 0.3) (layers "F.Cu" "B.Cu") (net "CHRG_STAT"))
 (segment (start 19.571 7.3947) (end 22.164 9.9877) (width 0.2) (layer "B.Cu") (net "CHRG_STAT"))
 (segment (start 19.571 4.7202) (end 19.571 7.3947) (width 0.2) (layer "B.Cu") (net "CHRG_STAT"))
 (segment (start 21.87 16.91) (end 21.87 21.2175) (width 0.2) (layer "F.Cu") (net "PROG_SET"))
 (segment (start 21.87 21.2175) (end 21.5875 21.5) (width 0.2) (layer "F.Cu") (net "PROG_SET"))
 (segment (start 23.14 11.09) (end 23.14 10.1883) (width 0.2) (layer "F.Cu") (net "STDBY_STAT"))
 (segment (start 23.7221 10.1883) (end 23.9428 9.9676) (width 0.2) (layer "F.Cu") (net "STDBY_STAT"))
 (segment (start 23.14 10.1883) (end 23.7221 10.1883) (width 0.2) (layer "F.Cu") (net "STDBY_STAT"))
 (segment (start 29.4104 4.5) (end 29.5625 4.5) (width 0.2) (layer "F.Cu") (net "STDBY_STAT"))
 (segment (start 28.6057 5.3047) (end 29.4104 4.5) (width 0.2) (layer "F.Cu") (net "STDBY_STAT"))
 (via (at 23.9428 9.9676) (size 0.6) (drill 0.3) (layers "F.Cu" "B.Cu") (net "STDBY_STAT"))
 (via (at 28.6057 5.3047) (size 0.6) (drill 0.3) (layers "F.Cu" "B.Cu") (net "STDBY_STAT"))
 (segment (start 28.6057 5.3047) (end 23.9428 9.9676) (width 0.2) (layer "B.Cu") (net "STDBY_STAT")))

